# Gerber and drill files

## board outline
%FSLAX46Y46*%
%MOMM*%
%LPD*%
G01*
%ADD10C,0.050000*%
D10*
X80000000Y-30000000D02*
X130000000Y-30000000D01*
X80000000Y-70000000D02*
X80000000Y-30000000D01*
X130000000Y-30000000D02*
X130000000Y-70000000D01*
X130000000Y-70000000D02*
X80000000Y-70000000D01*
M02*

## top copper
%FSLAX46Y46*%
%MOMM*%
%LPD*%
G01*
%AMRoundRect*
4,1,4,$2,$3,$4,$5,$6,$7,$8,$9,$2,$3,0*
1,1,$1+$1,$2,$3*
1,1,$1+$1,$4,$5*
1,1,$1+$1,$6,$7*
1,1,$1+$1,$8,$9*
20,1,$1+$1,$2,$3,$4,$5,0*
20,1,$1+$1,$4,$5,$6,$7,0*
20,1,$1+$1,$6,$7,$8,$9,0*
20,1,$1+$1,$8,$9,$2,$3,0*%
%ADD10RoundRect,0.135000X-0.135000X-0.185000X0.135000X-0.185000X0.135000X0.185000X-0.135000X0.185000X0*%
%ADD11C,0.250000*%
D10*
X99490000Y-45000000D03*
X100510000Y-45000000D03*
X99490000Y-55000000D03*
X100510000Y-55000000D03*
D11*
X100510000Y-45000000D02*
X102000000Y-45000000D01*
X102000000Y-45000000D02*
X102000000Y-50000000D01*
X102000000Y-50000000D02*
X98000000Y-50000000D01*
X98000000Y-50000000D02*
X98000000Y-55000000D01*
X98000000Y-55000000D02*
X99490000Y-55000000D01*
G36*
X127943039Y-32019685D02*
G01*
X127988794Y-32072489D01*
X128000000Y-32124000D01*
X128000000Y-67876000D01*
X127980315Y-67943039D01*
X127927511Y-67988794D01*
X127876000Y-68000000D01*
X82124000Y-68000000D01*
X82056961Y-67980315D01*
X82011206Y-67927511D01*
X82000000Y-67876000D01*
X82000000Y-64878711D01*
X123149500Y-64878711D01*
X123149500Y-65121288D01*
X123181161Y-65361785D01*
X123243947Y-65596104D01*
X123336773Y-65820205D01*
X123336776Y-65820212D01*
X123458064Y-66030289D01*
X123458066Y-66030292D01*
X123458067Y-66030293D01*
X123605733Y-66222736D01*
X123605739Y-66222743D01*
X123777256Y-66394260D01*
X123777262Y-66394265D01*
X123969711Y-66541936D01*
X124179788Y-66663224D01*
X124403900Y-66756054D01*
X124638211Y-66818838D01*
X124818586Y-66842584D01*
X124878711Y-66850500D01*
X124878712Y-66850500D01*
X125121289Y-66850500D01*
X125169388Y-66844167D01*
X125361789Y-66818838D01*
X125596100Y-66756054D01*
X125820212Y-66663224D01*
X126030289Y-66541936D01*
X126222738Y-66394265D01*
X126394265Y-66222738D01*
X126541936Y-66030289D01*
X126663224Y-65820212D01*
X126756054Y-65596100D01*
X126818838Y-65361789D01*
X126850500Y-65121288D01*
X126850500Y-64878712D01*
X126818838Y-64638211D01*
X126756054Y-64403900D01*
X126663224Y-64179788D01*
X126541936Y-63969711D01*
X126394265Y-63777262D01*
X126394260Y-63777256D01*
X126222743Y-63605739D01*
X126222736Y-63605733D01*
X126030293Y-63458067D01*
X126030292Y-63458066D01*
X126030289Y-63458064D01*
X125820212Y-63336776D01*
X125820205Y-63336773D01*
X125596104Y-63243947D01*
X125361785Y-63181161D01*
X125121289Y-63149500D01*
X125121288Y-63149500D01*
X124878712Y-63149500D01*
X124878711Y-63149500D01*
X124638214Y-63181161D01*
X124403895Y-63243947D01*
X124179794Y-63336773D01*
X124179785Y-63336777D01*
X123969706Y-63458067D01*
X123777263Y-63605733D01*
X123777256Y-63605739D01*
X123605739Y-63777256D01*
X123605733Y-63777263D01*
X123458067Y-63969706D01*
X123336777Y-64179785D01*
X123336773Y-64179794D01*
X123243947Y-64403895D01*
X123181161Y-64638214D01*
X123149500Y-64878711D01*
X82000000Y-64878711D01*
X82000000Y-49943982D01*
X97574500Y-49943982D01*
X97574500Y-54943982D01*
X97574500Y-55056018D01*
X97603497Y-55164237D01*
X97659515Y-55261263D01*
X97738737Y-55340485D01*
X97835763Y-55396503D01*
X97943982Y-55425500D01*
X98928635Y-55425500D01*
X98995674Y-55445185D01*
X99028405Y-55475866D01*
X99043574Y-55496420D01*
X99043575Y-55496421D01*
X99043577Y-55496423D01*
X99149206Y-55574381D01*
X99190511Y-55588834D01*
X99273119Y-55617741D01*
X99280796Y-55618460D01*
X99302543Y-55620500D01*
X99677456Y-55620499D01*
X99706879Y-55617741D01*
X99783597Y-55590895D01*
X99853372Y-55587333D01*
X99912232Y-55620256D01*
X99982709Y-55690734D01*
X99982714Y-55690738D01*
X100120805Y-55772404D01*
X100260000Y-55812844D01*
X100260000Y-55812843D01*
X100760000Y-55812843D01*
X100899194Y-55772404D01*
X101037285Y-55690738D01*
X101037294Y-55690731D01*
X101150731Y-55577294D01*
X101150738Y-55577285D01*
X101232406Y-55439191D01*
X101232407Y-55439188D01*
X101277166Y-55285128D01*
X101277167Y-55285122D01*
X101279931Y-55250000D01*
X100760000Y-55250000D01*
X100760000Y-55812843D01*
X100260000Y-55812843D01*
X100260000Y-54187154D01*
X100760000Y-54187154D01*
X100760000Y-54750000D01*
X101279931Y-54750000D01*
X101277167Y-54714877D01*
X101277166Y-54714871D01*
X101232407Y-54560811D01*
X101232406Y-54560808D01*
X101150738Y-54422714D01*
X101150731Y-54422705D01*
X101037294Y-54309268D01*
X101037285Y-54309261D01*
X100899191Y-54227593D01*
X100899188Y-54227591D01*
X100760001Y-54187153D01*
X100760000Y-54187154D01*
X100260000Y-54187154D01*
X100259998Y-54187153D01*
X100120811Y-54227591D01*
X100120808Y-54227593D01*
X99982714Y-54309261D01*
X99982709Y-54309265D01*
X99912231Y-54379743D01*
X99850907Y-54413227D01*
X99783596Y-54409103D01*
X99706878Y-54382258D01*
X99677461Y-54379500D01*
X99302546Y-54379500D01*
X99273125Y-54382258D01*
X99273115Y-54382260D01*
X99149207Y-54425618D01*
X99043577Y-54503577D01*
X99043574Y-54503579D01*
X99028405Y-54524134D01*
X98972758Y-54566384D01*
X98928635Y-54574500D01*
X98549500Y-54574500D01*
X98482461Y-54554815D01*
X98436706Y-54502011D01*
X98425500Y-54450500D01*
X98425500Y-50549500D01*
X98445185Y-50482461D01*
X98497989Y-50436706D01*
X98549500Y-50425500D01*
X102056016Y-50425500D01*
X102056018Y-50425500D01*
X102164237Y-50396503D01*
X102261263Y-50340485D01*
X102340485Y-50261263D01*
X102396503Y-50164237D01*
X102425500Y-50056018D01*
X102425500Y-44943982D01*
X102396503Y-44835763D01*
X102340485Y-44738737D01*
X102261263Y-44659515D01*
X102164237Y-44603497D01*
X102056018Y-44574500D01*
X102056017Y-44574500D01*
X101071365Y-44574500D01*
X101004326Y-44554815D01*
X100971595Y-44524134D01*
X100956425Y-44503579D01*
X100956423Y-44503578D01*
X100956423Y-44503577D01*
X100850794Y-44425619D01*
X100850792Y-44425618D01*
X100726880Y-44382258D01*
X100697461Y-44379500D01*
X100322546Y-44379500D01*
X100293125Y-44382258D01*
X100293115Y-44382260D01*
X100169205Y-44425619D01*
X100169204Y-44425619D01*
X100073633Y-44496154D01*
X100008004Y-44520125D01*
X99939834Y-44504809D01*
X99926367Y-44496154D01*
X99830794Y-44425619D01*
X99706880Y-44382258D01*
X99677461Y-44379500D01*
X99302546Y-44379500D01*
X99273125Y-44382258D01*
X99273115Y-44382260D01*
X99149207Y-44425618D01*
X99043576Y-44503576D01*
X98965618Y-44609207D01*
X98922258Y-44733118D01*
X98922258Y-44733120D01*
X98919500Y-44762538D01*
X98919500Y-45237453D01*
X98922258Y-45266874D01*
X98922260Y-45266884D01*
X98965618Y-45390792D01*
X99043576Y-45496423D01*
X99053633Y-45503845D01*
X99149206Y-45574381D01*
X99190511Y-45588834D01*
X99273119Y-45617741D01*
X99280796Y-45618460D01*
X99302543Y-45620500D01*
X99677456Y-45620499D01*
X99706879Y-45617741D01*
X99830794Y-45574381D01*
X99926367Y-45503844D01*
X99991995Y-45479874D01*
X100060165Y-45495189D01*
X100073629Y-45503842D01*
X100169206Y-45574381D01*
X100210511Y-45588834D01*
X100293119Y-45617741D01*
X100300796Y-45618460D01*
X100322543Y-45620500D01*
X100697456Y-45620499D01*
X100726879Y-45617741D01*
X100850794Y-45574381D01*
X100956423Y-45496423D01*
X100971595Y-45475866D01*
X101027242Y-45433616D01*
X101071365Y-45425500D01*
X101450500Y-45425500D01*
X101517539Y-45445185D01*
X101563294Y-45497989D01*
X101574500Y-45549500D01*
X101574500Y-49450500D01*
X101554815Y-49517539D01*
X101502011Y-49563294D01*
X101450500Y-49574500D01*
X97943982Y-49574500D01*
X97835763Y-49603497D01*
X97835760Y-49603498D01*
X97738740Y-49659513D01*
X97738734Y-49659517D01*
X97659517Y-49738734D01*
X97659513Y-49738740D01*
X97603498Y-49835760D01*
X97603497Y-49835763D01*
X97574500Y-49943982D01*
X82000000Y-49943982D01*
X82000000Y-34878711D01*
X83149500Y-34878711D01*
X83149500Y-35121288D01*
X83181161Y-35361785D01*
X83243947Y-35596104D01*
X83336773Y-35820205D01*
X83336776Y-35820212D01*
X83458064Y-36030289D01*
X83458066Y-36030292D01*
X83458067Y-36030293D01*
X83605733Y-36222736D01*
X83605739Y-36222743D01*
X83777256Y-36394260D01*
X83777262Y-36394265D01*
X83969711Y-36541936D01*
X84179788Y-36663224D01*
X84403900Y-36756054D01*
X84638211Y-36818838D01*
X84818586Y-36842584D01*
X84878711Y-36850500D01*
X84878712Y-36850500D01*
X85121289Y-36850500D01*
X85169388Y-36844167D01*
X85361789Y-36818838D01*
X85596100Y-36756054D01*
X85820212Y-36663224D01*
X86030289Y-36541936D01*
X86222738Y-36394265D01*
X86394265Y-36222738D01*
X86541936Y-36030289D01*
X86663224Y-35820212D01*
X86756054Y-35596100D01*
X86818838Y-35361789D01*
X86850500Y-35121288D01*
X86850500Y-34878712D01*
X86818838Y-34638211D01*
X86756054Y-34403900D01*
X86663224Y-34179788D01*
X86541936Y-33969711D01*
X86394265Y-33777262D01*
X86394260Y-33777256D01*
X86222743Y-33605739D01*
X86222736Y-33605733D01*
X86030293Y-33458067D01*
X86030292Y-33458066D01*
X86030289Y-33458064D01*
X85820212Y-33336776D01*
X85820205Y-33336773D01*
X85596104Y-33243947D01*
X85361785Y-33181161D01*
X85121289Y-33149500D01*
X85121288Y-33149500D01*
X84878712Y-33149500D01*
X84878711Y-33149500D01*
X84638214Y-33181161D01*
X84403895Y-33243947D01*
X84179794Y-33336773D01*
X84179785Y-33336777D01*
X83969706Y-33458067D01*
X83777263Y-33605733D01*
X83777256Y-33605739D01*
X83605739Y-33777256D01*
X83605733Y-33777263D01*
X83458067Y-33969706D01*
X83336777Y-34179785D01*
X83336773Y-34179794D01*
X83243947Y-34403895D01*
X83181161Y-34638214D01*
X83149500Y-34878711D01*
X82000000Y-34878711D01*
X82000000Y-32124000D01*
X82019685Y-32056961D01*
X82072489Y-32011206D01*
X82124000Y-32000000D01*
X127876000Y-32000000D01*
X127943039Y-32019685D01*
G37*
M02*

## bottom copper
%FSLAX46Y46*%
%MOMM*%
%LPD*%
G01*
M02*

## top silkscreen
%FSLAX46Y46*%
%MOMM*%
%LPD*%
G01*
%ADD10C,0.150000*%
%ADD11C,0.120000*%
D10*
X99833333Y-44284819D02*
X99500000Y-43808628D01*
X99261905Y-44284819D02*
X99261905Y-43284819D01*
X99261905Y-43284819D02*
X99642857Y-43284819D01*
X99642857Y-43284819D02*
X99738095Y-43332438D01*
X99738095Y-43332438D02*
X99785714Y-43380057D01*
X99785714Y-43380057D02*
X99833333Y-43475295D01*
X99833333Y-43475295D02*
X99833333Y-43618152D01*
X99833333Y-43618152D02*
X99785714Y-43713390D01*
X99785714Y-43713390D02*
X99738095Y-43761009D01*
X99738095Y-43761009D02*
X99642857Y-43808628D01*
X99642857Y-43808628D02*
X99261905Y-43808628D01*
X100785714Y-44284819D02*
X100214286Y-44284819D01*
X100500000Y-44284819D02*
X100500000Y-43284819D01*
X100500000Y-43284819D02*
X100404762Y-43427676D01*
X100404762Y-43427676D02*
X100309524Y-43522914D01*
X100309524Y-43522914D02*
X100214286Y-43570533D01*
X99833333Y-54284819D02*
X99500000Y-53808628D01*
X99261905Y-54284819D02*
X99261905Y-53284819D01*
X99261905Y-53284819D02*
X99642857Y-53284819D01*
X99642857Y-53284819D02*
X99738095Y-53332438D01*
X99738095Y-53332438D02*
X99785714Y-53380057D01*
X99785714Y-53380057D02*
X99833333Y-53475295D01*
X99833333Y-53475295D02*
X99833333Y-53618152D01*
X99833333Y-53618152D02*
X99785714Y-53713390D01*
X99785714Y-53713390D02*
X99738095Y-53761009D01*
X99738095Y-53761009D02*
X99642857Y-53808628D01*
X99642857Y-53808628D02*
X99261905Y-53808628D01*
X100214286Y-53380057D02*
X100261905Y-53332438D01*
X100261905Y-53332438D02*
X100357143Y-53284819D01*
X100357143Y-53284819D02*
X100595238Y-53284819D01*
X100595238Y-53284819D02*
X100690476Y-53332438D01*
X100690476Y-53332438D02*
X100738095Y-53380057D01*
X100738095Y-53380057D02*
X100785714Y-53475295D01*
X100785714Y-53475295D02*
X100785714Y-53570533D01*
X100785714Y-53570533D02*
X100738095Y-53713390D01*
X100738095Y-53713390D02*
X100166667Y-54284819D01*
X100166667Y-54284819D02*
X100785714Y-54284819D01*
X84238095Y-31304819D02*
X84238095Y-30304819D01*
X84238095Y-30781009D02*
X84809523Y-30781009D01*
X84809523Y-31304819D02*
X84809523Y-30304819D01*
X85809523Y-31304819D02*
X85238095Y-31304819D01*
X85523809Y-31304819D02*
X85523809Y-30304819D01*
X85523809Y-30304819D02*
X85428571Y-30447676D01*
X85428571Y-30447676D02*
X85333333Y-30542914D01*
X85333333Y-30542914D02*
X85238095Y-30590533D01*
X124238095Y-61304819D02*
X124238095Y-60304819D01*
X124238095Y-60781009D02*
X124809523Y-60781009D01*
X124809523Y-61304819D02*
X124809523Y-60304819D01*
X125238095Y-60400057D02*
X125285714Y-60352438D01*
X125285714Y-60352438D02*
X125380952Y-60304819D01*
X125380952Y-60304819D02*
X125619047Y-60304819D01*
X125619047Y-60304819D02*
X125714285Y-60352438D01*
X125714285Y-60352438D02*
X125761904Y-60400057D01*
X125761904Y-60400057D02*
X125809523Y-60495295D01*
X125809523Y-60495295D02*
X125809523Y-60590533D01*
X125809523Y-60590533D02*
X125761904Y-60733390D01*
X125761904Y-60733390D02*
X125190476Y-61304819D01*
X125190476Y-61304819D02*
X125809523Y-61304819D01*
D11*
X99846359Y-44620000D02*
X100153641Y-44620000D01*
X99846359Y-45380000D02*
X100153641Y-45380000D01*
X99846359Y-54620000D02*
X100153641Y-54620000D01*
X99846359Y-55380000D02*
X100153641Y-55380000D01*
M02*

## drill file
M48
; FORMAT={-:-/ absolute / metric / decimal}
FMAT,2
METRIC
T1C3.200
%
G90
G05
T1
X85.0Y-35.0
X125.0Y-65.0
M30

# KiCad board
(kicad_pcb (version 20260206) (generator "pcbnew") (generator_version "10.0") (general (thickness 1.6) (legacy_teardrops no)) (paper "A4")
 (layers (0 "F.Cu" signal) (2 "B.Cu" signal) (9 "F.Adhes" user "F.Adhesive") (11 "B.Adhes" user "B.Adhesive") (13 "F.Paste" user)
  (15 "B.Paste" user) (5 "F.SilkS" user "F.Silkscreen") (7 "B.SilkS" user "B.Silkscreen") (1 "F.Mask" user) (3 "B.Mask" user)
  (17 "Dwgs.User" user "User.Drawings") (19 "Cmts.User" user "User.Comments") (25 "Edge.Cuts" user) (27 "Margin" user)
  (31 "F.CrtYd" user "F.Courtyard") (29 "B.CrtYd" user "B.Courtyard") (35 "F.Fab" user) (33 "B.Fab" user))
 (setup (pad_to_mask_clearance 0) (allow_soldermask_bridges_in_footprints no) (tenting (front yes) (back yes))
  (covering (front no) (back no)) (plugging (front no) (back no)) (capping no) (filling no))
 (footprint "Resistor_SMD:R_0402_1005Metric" (layer "F.Cu") (at 100 45)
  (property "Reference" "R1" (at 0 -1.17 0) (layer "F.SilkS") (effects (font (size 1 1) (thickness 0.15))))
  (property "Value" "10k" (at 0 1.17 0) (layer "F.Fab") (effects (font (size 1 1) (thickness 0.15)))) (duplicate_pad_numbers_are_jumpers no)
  (fp_line (start -0.153641 -0.38) (end 0.153641 -0.38) (stroke (width 0.12) (type solid)) (layer "F.SilkS"))
  (fp_line (start -0.153641 0.38) (end 0.153641 0.38) (stroke (width 0.12) (type solid)) (layer "F.SilkS"))
  (pad "1" smd roundrect (at -0.51 0) (size 0.54 0.64) (layers "F.Cu" "F.Mask" "F.Paste") (roundrect_rratio 0.25) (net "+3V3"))
  (pad "2" smd roundrect (at 0.51 0) (size 0.54 0.64) (layers "F.Cu" "F.Mask" "F.Paste") (roundrect_rratio 0.25) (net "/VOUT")))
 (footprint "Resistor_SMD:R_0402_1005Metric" (layer "F.Cu") (at 100 55)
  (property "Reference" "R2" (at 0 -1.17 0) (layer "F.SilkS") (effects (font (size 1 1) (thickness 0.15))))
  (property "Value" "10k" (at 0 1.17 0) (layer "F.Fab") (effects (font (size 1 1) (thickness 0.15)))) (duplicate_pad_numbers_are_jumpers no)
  (fp_line (start -0.153641 -0.38) (end 0.153641 -0.38) (stroke (width 0.12) (type solid)) (layer "F.SilkS"))
  (fp_line (start -0.153641 0.38) (end 0.153641 0.38) (stroke (width 0.12) (type solid)) (layer "F.SilkS"))
  (pad "1" smd roundrect (at -0.51 0) (size 0.54 0.64) (layers "F.Cu" "F.Mask" "F.Paste") (roundrect_rratio 0.25) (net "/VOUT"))
  (pad "2" smd roundrect (at 0.51 0) (size 0.54 0.64) (layers "F.Cu" "F.Mask" "F.Paste") (roundrect_rratio 0.25) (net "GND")))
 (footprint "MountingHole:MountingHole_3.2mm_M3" (layer "F.Cu") (at 85 35)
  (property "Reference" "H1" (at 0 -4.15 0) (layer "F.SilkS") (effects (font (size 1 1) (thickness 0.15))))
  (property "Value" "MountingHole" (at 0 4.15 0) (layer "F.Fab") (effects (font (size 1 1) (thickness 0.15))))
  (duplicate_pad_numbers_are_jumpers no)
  (pad "" np_thru_hole circle (at 0 0) (size 3.2 3.2) (drill 3.2) (layers "*.Cu" "*.Mask")))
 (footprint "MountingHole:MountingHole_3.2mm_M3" (layer "F.Cu") (at 125 65)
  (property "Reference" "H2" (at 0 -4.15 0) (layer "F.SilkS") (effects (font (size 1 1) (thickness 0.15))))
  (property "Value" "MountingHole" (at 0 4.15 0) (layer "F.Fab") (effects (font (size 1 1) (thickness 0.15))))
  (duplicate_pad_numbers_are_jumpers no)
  (pad "" np_thru_hole circle (at 0 0) (size 3.2 3.2) (drill 3.2) (layers "*.Cu" "*.Mask")))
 (gr_line (start 80 30) (end 130 30) (stroke (width 0.05) (type default)) (layer "Edge.Cuts"))
 (gr_line (start 80 70) (end 80 30) (stroke (width 0.05) (type default)) (layer "Edge.Cuts"))
 (gr_line (start 130 30) (end 130 70) (stroke (width 0.05) (type default)) (layer "Edge.Cuts"))
 (gr_line (start 130 70) (end 80 70) (stroke (width 0.05) (type default)) (layer "Edge.Cuts"))
 (segment (start 100.51 45) (end 102 45) (width 0.25) (layer "F.Cu") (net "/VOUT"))
 (segment (start 102 45) (end 102 50) (width 0.25) (layer "F.Cu") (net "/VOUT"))
 (segment (start 102 50) (end 98 50) (width 0.25) (layer "F.Cu") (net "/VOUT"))
 (segment (start 98 50) (end 98 55) (width 0.25) (layer "F.Cu") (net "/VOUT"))
 (segment (start 98 55) (end 99.49 55) (width 0.25) (layer "F.Cu") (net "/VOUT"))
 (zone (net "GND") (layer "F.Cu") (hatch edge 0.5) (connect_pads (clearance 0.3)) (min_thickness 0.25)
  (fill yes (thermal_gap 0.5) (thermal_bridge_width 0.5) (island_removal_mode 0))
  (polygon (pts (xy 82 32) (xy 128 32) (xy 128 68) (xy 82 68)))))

